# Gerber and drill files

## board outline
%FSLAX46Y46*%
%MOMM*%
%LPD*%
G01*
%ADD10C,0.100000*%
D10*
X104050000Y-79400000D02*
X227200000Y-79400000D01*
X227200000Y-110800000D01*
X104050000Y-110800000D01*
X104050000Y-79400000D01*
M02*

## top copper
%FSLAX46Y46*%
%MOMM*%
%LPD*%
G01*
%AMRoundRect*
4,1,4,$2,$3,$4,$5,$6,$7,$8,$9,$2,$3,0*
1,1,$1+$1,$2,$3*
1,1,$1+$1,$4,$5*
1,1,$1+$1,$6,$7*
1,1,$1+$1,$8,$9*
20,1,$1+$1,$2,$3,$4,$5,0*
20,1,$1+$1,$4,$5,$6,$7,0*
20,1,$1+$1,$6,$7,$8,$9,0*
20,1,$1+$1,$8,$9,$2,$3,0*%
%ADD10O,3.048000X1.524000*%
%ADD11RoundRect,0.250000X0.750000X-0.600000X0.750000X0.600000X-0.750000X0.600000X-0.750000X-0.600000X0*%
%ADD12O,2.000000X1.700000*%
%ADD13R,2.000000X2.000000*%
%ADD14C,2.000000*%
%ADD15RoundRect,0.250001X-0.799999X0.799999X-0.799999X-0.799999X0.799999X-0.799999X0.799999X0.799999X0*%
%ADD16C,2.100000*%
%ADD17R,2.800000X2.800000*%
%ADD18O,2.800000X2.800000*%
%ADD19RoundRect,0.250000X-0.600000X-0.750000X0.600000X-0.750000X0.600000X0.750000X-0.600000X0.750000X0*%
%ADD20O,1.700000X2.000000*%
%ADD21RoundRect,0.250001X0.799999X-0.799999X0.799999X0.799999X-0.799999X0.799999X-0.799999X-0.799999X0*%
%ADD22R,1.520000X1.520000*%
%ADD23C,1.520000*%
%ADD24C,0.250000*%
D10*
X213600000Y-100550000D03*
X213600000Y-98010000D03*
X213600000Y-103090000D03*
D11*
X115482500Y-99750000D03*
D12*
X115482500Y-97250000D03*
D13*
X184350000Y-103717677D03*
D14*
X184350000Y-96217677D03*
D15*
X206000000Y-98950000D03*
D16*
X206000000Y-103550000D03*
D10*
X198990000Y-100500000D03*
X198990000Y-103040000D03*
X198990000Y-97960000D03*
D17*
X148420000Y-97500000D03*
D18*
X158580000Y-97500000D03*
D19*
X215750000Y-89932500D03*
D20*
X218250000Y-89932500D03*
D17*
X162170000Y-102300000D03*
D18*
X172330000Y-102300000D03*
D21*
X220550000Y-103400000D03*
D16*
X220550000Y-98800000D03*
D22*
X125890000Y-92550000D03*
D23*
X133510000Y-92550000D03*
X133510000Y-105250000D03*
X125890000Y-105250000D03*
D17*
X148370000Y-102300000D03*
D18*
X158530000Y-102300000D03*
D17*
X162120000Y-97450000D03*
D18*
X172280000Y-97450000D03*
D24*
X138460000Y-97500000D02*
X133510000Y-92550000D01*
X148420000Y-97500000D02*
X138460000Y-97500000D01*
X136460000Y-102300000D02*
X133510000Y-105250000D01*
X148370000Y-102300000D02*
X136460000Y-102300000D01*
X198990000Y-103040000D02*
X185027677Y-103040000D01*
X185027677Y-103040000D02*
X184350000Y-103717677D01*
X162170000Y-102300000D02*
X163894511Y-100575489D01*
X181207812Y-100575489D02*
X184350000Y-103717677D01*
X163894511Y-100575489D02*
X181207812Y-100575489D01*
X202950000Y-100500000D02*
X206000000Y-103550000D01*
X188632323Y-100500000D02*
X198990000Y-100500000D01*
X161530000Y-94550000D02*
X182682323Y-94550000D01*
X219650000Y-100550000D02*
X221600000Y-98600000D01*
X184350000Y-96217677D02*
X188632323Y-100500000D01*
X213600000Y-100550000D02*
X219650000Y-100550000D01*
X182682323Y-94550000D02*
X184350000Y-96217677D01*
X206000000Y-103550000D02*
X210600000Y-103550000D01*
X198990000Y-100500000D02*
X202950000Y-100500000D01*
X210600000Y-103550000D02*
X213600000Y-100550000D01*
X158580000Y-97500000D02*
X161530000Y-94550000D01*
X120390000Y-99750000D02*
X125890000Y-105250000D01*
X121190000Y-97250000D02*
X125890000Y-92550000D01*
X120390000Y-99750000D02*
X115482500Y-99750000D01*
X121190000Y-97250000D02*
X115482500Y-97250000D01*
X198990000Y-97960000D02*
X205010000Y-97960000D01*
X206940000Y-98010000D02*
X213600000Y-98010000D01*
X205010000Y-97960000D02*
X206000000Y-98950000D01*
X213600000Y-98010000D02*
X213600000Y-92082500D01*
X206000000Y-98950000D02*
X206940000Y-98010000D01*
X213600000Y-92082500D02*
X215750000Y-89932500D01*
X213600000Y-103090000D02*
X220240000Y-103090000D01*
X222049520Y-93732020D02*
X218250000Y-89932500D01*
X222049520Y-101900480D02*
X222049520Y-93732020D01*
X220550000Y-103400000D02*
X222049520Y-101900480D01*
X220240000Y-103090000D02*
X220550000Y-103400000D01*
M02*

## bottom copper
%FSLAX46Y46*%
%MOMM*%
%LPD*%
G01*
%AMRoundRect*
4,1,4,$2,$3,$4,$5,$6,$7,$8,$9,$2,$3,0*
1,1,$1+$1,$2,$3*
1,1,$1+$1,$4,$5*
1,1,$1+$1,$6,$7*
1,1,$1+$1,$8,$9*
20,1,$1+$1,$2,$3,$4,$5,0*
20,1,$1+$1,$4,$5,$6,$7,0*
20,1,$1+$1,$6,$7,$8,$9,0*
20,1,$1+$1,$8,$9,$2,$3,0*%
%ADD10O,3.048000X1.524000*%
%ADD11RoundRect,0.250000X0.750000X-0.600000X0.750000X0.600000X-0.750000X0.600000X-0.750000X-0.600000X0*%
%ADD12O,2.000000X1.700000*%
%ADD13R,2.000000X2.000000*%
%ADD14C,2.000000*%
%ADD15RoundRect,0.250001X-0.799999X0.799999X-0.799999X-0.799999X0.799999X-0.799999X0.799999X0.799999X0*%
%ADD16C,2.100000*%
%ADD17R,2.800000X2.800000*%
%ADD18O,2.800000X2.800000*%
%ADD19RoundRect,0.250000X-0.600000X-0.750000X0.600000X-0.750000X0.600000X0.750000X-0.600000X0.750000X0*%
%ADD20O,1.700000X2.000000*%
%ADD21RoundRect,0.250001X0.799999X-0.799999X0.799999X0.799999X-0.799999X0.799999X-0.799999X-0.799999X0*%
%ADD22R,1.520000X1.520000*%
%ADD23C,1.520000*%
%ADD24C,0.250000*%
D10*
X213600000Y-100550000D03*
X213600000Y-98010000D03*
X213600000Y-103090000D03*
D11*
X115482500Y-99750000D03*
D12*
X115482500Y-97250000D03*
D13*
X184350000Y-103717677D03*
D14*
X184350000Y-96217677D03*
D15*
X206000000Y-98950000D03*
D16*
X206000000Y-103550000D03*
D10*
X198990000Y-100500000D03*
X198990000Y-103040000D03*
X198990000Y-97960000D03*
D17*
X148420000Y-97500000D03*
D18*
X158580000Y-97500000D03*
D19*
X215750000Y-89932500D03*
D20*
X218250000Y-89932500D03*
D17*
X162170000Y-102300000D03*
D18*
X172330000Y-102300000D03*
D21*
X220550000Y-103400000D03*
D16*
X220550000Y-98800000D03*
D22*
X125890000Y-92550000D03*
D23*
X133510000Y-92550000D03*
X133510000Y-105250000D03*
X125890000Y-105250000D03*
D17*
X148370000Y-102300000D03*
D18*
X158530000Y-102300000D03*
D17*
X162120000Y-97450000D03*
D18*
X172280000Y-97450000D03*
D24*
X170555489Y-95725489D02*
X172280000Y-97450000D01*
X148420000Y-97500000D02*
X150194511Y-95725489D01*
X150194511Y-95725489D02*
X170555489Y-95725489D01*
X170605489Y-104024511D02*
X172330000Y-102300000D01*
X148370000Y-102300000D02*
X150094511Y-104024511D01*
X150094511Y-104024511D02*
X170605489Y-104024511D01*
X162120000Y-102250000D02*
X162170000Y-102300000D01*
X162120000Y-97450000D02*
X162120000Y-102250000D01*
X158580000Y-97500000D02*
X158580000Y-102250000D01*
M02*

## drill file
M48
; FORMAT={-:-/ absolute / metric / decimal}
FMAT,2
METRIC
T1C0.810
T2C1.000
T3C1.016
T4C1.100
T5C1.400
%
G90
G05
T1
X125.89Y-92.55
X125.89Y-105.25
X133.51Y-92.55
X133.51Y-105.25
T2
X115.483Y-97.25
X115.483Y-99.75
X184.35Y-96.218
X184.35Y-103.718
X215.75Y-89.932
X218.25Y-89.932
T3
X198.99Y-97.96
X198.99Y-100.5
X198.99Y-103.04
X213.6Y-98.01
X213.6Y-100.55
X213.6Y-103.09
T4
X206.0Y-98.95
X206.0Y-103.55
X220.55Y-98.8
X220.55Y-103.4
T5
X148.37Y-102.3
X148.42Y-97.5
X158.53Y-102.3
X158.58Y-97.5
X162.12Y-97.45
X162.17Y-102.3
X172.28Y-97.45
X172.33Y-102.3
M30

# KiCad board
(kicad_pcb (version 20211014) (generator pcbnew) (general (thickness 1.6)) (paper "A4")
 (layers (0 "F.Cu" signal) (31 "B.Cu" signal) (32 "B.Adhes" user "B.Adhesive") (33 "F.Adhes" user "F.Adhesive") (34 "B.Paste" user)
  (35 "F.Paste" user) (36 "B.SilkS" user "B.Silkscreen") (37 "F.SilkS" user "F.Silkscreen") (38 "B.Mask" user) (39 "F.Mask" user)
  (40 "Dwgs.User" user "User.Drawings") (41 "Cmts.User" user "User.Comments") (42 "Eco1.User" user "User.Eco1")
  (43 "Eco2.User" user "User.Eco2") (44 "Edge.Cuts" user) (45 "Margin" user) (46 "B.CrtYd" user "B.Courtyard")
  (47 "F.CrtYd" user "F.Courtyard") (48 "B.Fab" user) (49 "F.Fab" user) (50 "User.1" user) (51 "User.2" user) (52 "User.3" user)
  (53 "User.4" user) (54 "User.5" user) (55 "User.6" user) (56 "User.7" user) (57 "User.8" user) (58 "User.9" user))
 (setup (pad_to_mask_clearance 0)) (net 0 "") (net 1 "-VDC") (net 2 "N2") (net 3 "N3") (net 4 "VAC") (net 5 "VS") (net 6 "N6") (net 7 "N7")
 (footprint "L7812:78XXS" (layer "F.Cu") (at 216.14 100.55 -90)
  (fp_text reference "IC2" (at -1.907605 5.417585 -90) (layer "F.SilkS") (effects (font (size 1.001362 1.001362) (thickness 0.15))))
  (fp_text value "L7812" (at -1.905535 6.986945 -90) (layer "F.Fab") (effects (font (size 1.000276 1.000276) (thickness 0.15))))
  (pad "GND" thru_hole oval locked (at 0 2.54 270) (size 1.524 3.048) (drill 1.016) (layers *.Cu *.Mask) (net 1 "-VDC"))
  (pad "IN" thru_hole oval locked (at -2.54 2.54 270) (size 1.524 3.048) (drill 1.016) (layers *.Cu *.Mask) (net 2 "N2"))
  (pad "OUT" thru_hole oval locked (at 2.54 2.54 270) (size 1.524 3.048) (drill 1.016) (layers *.Cu *.Mask) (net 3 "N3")))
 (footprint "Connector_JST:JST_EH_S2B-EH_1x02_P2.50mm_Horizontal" (layer "F.Cu") (at 115.4825 99.75 90)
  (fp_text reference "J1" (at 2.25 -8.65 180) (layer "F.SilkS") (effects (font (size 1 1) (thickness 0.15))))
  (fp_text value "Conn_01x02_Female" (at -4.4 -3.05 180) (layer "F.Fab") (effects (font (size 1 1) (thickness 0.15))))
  (pad "1" thru_hole roundrect (at 0 0 90) (size 1.7 2) (drill 1) (layers *.Cu *.Mask) (roundrect_rratio 0.147059) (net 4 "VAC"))
  (pad "2" thru_hole oval (at 2.5 0 90) (size 1.7 2) (drill 1) (layers *.Cu *.Mask) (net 4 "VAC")))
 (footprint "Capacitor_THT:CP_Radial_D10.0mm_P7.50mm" (layer "F.Cu") (at 184.35 103.717677 90)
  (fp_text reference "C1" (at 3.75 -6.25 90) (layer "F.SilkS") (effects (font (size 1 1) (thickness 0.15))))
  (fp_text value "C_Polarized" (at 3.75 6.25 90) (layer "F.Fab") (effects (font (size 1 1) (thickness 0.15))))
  (pad "1" thru_hole rect (at 0 0 90) (size 2 2) (drill 1) (layers *.Cu *.Mask) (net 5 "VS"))
  (pad "2" thru_hole circle (at 7.5 0 90) (size 2 2) (drill 1) (layers *.Cu *.Mask) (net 1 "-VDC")))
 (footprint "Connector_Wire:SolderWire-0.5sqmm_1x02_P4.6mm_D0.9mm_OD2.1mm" (layer "F.Cu") (at 206 98.95 -90)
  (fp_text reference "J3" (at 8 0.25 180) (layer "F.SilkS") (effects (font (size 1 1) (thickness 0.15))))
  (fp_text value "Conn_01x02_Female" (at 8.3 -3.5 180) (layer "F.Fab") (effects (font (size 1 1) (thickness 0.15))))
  (pad "1" thru_hole roundrect (at 0 0 270) (size 2.1 2.1) (drill 1.1) (layers *.Cu *.Mask) (roundrect_rratio 0.119048) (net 2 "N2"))
  (pad "2" thru_hole circle (at 4.6 0 270) (size 2.1 2.1) (drill 1.1) (layers *.Cu *.Mask) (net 1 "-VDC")))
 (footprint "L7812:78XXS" (layer "F.Cu") (at 196.45 100.5 90)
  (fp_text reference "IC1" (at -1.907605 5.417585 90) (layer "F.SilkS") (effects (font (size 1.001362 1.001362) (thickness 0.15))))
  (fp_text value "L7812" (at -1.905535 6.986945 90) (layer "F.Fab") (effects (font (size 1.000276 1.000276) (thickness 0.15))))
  (pad "GND" thru_hole oval locked (at 0 2.54 90) (size 1.524 3.048) (drill 1.016) (layers *.Cu *.Mask) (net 1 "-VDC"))
  (pad "IN" thru_hole oval locked (at -2.54 2.54 90) (size 1.524 3.048) (drill 1.016) (layers *.Cu *.Mask) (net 5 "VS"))
  (pad "OUT" thru_hole oval locked (at 2.54 2.54 90) (size 1.524 3.048) (drill 1.016) (layers *.Cu *.Mask) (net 2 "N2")))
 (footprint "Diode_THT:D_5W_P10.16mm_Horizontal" (layer "F.Cu") (at 148.42 97.5)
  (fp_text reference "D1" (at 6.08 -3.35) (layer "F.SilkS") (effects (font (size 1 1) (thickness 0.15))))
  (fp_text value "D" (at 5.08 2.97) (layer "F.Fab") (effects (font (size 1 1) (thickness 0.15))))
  (pad "1" thru_hole rect (at 0 0) (size 2.8 2.8) (drill 1.4) (layers *.Cu *.Mask) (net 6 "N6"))
  (pad "2" thru_hole oval (at 10.16 0) (size 2.8 2.8) (drill 1.4) (layers *.Cu *.Mask) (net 1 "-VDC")))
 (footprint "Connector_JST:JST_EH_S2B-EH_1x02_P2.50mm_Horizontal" (layer "F.Cu") (at 215.75 89.9325)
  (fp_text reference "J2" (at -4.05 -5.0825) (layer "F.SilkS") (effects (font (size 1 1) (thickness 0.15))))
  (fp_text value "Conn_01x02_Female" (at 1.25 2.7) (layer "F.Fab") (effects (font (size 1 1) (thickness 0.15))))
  (pad "1" thru_hole roundrect (at 0 0) (size 1.7 2) (drill 1) (layers *.Cu *.Mask) (roundrect_rratio 0.147059) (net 2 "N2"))
  (pad "2" thru_hole oval (at 2.5 0) (size 1.7 2) (drill 1) (layers *.Cu *.Mask) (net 3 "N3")))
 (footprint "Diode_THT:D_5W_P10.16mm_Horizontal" (layer "F.Cu") (at 162.17 102.3)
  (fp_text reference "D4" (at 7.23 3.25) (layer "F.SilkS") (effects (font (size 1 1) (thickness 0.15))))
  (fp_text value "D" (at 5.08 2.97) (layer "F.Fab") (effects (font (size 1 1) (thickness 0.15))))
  (pad "1" thru_hole rect (at 0 0) (size 2.8 2.8) (drill 1.4) (layers *.Cu *.Mask) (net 5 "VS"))
  (pad "2" thru_hole oval (at 10.16 0) (size 2.8 2.8) (drill 1.4) (layers *.Cu *.Mask) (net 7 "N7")))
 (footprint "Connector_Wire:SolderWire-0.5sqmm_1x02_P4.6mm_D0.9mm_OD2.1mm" (layer "F.Cu") (at 220.55 103.4 90)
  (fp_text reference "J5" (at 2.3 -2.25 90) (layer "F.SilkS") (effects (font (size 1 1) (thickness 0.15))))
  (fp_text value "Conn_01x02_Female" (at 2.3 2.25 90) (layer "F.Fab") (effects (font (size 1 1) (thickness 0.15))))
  (pad "1" thru_hole roundrect (at 0 0 90) (size 2.1 2.1) (drill 1.1) (layers *.Cu *.Mask) (roundrect_rratio 0.119048) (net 3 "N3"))
  (pad "2" thru_hole circle (at 4.6 0 90) (size 2.1 2.1) (drill 1.1) (layers *.Cu *.Mask) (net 1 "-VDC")))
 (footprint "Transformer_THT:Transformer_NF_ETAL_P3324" (layer "F.Cu") (at 125.89 92.55 90)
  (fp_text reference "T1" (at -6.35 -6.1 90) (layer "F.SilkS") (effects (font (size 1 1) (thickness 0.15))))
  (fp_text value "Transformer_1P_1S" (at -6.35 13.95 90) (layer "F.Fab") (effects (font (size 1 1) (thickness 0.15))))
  (pad "1" thru_hole rect (at 0 0 90) (size 1.52 1.52) (drill 0.81) (layers *.Cu *.Mask) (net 4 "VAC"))
  (pad "3" thru_hole circle (at 0 7.62 90) (size 1.52 1.52) (drill 0.81) (layers *.Cu *.Mask) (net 6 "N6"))
  (pad "4" thru_hole circle (at -12.7 7.62 90) (size 1.52 1.52) (drill 0.81) (layers *.Cu *.Mask) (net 7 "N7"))
  (pad "6" thru_hole circle (at -12.7 0 90) (size 1.52 1.52) (drill 0.81) (layers *.Cu *.Mask) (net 4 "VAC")))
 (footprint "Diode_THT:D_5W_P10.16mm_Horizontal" (layer "F.Cu") (at 148.37 102.3)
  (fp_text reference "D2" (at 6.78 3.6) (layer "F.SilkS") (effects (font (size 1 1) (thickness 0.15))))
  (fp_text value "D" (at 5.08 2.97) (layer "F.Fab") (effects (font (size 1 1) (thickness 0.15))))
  (pad "1" thru_hole rect (at 0 0) (size 2.8 2.8) (drill 1.4) (layers *.Cu *.Mask) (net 7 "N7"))
  (pad "2" thru_hole oval (at 10.16 0) (size 2.8 2.8) (drill 1.4) (layers *.Cu *.Mask) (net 1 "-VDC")))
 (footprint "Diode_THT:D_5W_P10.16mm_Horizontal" (layer "F.Cu") (at 162.12 97.45)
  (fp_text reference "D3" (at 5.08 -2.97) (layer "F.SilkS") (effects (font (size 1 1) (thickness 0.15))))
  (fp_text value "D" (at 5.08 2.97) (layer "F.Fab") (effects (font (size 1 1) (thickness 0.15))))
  (pad "1" thru_hole rect (at 0 0) (size 2.8 2.8) (drill 1.4) (layers *.Cu *.Mask) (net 5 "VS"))
  (pad "2" thru_hole oval (at 10.16 0) (size 2.8 2.8) (drill 1.4) (layers *.Cu *.Mask) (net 6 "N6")))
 (gr_rect (start 104.05 79.4) (end 227.2 110.8) (layer "Edge.Cuts") (width 0.1) (fill none))
 (segment (start 138.46 97.5) (end 133.51 92.55) (width 0.25) (layer "F.Cu") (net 6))
 (segment (start 148.42 97.5) (end 138.46 97.5) (width 0.25) (layer "F.Cu") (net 6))
 (segment (start 170.555489 95.725489) (end 172.28 97.45) (width 0.25) (layer "B.Cu") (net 6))
 (segment (start 148.42 97.5) (end 150.194511 95.725489) (width 0.25) (layer "B.Cu") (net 6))
 (segment (start 150.194511 95.725489) (end 170.555489 95.725489) (width 0.25) (layer "B.Cu") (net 6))
 (segment (start 136.46 102.3) (end 133.51 105.25) (width 0.25) (layer "F.Cu") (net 7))
 (segment (start 148.37 102.3) (end 136.46 102.3) (width 0.25) (layer "F.Cu") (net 7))
 (segment (start 170.605489 104.024511) (end 172.33 102.3) (width 0.25) (layer "B.Cu") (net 7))
 (segment (start 148.37 102.3) (end 150.094511 104.024511) (width 0.25) (layer "B.Cu") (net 7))
 (segment (start 150.094511 104.024511) (end 170.605489 104.024511) (width 0.25) (layer "B.Cu") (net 7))
 (segment (start 198.99 103.04) (end 185.027677 103.04) (width 0.25) (layer "F.Cu") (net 5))
 (segment (start 185.027677 103.04) (end 184.35 103.717677) (width 0.25) (layer "F.Cu") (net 5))
 (segment (start 162.17 102.3) (end 163.894511 100.575489) (width 0.25) (layer "F.Cu") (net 5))
 (segment (start 181.207812 100.575489) (end 184.35 103.717677) (width 0.25) (layer "F.Cu") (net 5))
 (segment (start 163.894511 100.575489) (end 181.207812 100.575489) (width 0.25) (layer "F.Cu") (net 5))
 (segment (start 162.12 102.25) (end 162.17 102.3) (width 0.25) (layer "B.Cu") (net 5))
 (segment (start 162.12 97.45) (end 162.12 102.25) (width 0.25) (layer "B.Cu") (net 5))
 (segment (start 202.95 100.5) (end 206 103.55) (width 0.25) (layer "F.Cu") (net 1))
 (segment (start 188.632323 100.5) (end 198.99 100.5) (width 0.25) (layer "F.Cu") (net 1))
 (segment (start 161.53 94.55) (end 182.682323 94.55) (width 0.25) (layer "F.Cu") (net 1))
 (segment (start 219.65 100.55) (end 221.6 98.6) (width 0.25) (layer "F.Cu") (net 1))
 (segment (start 184.35 96.217677) (end 188.632323 100.5) (width 0.25) (layer "F.Cu") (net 1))
 (segment (start 213.6 100.55) (end 219.65 100.55) (width 0.25) (layer "F.Cu") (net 1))
 (segment (start 182.682323 94.55) (end 184.35 96.217677) (width 0.25) (layer "F.Cu") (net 1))
 (segment (start 206 103.55) (end 210.6 103.55) (width 0.25) (layer "F.Cu") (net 1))
 (segment (start 198.99 100.5) (end 202.95 100.5) (width 0.25) (layer "F.Cu") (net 1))
 (segment (start 210.6 103.55) (end 213.6 100.55) (width 0.25) (layer "F.Cu") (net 1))
 (segment (start 158.58 97.5) (end 161.53 94.55) (width 0.25) (layer "F.Cu") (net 1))
 (segment (start 158.58 97.5) (end 158.58 102.25) (width 0.25) (layer "B.Cu") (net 1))
 (segment (start 120.39 99.75) (end 125.89 105.25) (width 0.25) (layer "F.Cu") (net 4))
 (segment (start 121.19 97.25) (end 125.89 92.55) (width 0.25) (layer "F.Cu") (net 4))
 (segment (start 120.39 99.75) (end 115.4825 99.75) (width 0.25) (layer "F.Cu") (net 4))
 (segment (start 121.19 97.25) (end 115.4825 97.25) (width 0.25) (layer "F.Cu") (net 4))
 (segment (start 198.99 97.96) (end 205.01 97.96) (width 0.25) (layer "F.Cu") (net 2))
 (segment (start 206.94 98.01) (end 213.6 98.01) (width 0.25) (layer "F.Cu") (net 2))
 (segment (start 205.01 97.96) (end 206 98.95) (width 0.25) (layer "F.Cu") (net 2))
 (segment (start 213.6 98.01) (end 213.6 92.0825) (width 0.25) (layer "F.Cu") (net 2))
 (segment (start 206 98.95) (end 206.94 98.01) (width 0.25) (layer "F.Cu") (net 2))
 (segment (start 213.6 92.0825) (end 215.75 89.9325) (width 0.25) (layer "F.Cu") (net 2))
 (segment (start 213.6 103.09) (end 220.24 103.09) (width 0.25) (layer "F.Cu") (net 3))
 (segment (start 222.04952 93.73202) (end 218.25 89.9325) (width 0.25) (layer "F.Cu") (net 3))
 (segment (start 222.04952 101.90048) (end 222.04952 93.73202) (width 0.25) (layer "F.Cu") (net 3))
 (segment (start 220.55 103.4) (end 222.04952 101.90048) (width 0.25) (layer "F.Cu") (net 3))
 (segment (start 220.24 103.09) (end 220.55 103.4) (width 0.25) (layer "F.Cu") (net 3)))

